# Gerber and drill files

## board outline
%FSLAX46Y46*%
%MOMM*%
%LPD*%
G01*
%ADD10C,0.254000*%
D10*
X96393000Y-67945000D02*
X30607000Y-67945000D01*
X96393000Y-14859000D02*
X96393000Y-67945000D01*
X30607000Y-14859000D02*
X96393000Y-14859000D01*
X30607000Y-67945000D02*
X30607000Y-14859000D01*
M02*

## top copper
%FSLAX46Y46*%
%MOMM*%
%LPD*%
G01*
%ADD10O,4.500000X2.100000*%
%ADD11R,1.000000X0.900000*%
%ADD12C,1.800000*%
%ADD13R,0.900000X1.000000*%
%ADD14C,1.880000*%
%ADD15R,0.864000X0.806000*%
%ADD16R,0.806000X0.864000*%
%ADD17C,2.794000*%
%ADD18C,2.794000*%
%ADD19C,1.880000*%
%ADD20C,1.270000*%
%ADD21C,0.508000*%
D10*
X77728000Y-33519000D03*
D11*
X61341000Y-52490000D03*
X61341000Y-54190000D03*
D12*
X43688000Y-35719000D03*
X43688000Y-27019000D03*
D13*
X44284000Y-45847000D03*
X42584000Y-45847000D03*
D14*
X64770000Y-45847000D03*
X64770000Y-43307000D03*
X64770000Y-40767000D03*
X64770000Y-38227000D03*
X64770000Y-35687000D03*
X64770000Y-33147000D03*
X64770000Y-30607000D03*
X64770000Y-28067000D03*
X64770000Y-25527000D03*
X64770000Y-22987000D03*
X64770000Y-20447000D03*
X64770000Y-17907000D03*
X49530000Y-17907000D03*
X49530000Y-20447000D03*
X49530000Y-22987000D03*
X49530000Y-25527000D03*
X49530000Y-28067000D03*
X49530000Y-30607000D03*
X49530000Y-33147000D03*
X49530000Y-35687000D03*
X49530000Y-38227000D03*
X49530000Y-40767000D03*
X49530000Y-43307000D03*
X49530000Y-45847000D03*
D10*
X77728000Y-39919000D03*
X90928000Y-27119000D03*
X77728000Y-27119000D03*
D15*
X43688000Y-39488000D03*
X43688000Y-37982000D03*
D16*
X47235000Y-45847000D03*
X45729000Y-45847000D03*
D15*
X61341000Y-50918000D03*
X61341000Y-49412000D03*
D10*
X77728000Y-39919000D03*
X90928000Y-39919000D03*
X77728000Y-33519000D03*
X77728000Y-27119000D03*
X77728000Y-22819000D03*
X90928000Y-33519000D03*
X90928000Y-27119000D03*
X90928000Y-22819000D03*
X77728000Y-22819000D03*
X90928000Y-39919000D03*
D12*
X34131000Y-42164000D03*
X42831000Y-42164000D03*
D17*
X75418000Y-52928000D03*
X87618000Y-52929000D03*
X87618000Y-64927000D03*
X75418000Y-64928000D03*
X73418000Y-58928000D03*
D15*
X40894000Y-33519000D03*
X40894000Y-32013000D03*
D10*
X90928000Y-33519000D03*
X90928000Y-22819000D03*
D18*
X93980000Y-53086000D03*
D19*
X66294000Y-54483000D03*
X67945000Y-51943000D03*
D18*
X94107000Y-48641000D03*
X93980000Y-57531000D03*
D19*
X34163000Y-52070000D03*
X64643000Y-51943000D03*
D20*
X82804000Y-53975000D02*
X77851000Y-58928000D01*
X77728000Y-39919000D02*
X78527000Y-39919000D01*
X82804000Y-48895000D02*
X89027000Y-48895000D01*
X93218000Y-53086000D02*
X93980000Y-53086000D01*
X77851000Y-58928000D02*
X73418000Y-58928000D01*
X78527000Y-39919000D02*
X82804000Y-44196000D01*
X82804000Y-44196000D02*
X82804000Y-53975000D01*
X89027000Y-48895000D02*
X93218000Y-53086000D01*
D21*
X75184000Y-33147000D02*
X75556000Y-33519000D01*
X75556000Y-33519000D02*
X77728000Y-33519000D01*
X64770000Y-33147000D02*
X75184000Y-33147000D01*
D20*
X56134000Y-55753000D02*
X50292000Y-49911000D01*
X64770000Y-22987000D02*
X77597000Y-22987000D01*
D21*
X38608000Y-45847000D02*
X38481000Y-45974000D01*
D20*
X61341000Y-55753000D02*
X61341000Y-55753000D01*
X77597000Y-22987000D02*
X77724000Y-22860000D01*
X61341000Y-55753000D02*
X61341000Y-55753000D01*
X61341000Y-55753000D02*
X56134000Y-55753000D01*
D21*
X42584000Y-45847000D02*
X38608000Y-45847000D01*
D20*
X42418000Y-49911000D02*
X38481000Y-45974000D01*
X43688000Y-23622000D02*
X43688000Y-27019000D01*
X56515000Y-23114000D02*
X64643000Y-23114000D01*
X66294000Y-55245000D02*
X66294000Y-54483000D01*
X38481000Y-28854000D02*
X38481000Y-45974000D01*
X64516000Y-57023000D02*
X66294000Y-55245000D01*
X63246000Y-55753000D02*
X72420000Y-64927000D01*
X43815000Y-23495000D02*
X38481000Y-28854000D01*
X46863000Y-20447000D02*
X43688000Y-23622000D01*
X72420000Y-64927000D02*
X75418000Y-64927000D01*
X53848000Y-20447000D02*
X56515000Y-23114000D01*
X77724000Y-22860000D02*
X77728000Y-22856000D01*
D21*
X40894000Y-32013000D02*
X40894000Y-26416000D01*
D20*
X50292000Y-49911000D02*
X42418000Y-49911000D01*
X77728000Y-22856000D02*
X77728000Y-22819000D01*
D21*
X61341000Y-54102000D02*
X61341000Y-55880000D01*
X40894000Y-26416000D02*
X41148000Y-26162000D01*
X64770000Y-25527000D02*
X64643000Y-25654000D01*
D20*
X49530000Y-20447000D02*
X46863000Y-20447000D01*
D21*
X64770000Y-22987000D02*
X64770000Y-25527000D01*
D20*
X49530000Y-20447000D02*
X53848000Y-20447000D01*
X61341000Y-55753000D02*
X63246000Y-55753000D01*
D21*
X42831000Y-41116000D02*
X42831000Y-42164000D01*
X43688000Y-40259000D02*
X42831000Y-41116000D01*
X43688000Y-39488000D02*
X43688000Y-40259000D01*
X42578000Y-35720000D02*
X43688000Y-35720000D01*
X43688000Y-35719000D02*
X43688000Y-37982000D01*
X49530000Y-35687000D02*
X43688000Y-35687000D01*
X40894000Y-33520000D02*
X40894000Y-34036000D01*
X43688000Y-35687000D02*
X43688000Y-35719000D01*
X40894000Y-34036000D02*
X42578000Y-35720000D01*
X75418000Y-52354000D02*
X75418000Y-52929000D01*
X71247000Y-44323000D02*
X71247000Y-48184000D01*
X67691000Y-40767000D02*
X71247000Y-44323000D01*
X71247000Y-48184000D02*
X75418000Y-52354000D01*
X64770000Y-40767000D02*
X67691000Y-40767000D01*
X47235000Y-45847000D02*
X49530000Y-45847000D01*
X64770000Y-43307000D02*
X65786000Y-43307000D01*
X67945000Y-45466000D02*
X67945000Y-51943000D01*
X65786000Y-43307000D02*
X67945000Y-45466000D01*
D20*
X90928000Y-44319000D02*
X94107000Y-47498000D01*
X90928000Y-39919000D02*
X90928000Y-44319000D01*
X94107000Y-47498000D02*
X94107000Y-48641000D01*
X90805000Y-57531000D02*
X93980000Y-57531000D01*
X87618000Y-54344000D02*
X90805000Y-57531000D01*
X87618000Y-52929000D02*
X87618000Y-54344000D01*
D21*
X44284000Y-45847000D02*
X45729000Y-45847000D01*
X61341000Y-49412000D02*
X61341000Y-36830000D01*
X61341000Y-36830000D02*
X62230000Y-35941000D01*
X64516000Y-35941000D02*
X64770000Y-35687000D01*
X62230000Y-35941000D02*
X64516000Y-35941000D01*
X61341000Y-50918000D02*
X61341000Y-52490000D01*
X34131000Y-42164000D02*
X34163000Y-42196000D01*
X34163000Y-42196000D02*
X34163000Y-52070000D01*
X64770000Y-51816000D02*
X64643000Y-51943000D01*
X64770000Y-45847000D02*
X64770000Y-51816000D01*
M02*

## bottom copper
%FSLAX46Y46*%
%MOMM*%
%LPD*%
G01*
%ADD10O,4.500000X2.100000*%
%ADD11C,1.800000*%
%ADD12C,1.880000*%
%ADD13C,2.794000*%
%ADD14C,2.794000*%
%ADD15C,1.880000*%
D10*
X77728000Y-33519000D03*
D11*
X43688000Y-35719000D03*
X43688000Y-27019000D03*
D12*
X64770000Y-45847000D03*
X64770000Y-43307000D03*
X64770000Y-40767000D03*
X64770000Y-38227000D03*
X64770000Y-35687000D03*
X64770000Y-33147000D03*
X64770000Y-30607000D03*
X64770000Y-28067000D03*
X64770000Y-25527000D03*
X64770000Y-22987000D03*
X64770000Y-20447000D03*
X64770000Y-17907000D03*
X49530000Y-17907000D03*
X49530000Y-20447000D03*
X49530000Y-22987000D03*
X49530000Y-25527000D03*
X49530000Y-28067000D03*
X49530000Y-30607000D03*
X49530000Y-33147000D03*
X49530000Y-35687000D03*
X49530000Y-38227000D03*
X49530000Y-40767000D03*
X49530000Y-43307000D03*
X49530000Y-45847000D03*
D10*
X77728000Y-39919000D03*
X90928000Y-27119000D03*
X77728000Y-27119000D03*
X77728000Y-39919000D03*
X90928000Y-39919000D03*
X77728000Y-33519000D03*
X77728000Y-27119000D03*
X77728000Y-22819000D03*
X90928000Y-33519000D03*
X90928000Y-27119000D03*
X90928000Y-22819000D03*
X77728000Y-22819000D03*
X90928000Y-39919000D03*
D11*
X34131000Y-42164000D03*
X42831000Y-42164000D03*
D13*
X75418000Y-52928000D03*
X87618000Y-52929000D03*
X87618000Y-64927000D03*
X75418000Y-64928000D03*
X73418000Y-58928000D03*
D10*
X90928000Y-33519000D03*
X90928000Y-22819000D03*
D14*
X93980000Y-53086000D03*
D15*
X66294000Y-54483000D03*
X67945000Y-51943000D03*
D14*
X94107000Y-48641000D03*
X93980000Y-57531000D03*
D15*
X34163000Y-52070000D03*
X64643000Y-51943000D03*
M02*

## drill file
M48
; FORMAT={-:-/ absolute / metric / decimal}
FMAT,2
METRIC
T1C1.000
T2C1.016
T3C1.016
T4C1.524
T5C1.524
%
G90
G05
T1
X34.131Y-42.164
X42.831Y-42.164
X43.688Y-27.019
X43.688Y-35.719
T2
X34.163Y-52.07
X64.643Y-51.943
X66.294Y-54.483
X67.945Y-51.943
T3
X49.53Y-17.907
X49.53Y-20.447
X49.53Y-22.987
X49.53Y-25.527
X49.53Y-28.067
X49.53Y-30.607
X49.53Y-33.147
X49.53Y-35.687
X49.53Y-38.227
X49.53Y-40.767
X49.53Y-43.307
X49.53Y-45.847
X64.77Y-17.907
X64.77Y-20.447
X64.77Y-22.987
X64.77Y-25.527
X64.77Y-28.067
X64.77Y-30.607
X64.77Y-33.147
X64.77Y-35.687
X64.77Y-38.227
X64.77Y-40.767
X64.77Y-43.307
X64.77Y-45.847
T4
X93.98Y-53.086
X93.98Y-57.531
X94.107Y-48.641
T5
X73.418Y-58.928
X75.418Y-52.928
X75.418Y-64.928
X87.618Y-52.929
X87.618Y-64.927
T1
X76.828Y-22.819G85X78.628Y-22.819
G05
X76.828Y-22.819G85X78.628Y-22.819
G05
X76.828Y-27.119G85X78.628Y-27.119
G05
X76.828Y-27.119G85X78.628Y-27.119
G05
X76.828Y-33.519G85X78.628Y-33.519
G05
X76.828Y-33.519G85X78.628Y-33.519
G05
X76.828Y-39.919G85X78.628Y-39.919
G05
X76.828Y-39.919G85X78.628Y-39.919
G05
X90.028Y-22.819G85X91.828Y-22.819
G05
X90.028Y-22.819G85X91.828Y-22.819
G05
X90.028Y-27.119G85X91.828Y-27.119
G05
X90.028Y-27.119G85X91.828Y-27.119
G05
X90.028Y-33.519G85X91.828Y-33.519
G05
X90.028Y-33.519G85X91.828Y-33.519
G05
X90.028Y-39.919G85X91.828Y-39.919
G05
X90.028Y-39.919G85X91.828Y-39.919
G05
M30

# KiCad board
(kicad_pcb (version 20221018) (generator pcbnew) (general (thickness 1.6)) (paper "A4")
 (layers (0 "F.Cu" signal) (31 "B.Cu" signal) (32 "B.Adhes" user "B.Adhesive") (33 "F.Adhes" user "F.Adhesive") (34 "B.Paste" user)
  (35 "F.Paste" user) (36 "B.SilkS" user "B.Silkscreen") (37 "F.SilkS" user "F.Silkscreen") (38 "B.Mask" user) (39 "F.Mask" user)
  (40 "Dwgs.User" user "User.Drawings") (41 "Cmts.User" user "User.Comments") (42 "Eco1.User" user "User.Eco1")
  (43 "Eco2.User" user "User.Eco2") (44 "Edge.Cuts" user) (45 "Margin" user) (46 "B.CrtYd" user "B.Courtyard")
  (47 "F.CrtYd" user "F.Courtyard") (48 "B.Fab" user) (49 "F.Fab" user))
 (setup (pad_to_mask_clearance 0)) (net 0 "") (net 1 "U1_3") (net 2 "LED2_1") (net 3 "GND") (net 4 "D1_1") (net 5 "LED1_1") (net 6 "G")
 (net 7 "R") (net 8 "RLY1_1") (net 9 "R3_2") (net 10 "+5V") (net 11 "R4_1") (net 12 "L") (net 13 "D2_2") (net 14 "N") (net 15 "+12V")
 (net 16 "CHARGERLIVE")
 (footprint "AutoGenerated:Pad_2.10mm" (layer "F.Cu") (at 77.728 33.519)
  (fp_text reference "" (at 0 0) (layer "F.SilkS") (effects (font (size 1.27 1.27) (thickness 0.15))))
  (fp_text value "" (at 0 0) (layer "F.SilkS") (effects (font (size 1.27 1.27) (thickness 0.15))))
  (pad "5" thru_hole oval (at 0 0 90) (size 2.1 4.5) (drill oval 1 2.8) (layers "*.Cu" "*.Paste" "*.Mask") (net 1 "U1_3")))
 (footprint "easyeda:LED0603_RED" (layer "F.Cu") (at 61.341 53.34 -90)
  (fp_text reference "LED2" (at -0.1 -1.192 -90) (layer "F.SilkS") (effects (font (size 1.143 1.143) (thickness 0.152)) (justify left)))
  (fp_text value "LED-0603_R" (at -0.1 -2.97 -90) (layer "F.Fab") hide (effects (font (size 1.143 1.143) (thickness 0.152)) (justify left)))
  (pad "1" smd rect (at -0.85 0 180) (size 1 0.9) (layers "F.Cu" "F.Paste" "F.Mask") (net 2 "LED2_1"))
  (pad "2" smd rect (at 0.85 0 180) (size 1 0.9) (layers "F.Cu" "F.Paste" "F.Mask") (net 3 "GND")))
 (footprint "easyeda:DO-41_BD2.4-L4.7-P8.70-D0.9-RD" (layer "F.Cu") (at 43.688 31.369 -90)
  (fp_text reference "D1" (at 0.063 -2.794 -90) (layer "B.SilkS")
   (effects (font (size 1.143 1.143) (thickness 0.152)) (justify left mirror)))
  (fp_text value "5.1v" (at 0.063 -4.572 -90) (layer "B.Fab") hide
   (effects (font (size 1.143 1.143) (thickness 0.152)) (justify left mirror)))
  (pad "1" thru_hole circle (at 4.35 0 270) (size 1.8 1.8) (drill 1) (layers "*.Cu" "*.Paste" "*.Mask") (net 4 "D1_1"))
  (pad "2" thru_hole circle (at -4.35 0 270) (size 1.8 1.8) (drill 1) (layers "*.Cu" "*.Paste" "*.Mask") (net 3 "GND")))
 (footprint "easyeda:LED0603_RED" (layer "F.Cu") (at 43.434 45.847 180)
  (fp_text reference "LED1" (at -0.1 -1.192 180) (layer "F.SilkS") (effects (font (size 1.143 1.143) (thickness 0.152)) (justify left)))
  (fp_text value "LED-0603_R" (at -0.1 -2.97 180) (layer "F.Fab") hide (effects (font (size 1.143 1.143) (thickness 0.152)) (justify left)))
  (pad "1" smd rect (at -0.85 0 90) (size 1 0.9) (layers "F.Cu" "F.Paste" "F.Mask") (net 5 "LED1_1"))
  (pad "2" smd rect (at 0.85 0 90) (size 1 0.9) (layers "F.Cu" "F.Paste" "F.Mask") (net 3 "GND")))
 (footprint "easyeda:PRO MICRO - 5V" (layer "F.Cu") (at 57.15 31.877)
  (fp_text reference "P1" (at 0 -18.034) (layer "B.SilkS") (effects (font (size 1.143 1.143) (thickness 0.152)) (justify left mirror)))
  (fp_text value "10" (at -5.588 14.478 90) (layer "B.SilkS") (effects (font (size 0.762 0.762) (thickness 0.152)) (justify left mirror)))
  (pad "1" thru_hole circle (at 7.62 13.97) (size 1.88 1.88) (drill 1.016) (layers "*.Cu" "*.Paste" "*.Mask") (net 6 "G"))
  (pad "2" thru_hole circle (at 7.62 11.43) (size 1.88 1.88) (drill 1.016) (layers "*.Cu" "*.Paste" "*.Mask") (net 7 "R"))
  (pad "3" thru_hole circle (at 7.62 8.89) (size 1.88 1.88) (drill 1.016) (layers "*.Cu" "*.Paste" "*.Mask") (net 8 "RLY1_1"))
  (pad "4" thru_hole circle (at 7.62 6.35) (size 1.88 1.88) (drill 1.016) (layers "*.Cu" "*.Paste" "*.Mask"))
  (pad "5" thru_hole circle (at 7.62 3.81) (size 1.88 1.88) (drill 1.016) (layers "*.Cu" "*.Paste" "*.Mask") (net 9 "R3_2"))
  (pad "6" thru_hole circle (at 7.62 1.27) (size 1.88 1.88) (drill 1.016) (layers "*.Cu" "*.Paste" "*.Mask") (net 1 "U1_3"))
  (pad "7" thru_hole circle (at 7.62 -1.27) (size 1.88 1.88) (drill 1.016) (layers "*.Cu" "*.Paste" "*.Mask"))
  (pad "8" thru_hole circle (at 7.62 -3.81) (size 1.88 1.88) (drill 1.016) (layers "*.Cu" "*.Paste" "*.Mask"))
  (pad "9" thru_hole circle (at 7.62 -6.35) (size 1.88 1.88) (drill 1.016) (layers "*.Cu" "*.Paste" "*.Mask") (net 3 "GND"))
  (pad "10" thru_hole circle (at 7.62 -8.89) (size 1.88 1.88) (drill 1.016) (layers "*.Cu" "*.Paste" "*.Mask") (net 3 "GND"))
  (pad "11" thru_hole circle (at 7.62 -11.43) (size 1.88 1.88) (drill 1.016) (layers "*.Cu" "*.Paste" "*.Mask"))
  (pad "12" thru_hole circle (at 7.62 -13.97) (size 1.88 1.88) (drill 1.016) (layers "*.Cu" "*.Paste" "*.Mask"))
  (pad "13" thru_hole circle (at -7.62 -13.97 180) (size 1.88 1.88) (drill 1.016) (layers "*.Cu" "*.Paste" "*.Mask"))
  (pad "14" thru_hole circle (at -7.62 -11.43 180) (size 1.88 1.88) (drill 1.016) (layers "*.Cu" "*.Paste" "*.Mask") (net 3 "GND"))
  (pad "15" thru_hole circle (at -7.62 -8.89 180) (size 1.88 1.88) (drill 1.016) (layers "*.Cu" "*.Paste" "*.Mask"))
  (pad "16" thru_hole circle (at -7.62 -6.35 180) (size 1.88 1.88) (drill 1.016) (layers "*.Cu" "*.Paste" "*.Mask") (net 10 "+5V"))
  (pad "17" thru_hole circle (at -7.62 -3.81 180) (size 1.88 1.88) (drill 1.016) (layers "*.Cu" "*.Paste" "*.Mask"))
  (pad "18" thru_hole circle (at -7.62 -1.27 180) (size 1.88 1.88) (drill 1.016) (layers "*.Cu" "*.Paste" "*.Mask"))
  (pad "19" thru_hole circle (at -7.62 1.27 180) (size 1.88 1.88) (drill 1.016) (layers "*.Cu" "*.Paste" "*.Mask"))
  (pad "20" thru_hole circle (at -7.62 3.81 180) (size 1.88 1.88) (drill 1.016) (layers "*.Cu" "*.Paste" "*.Mask") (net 4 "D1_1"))
  (pad "21" thru_hole circle (at -7.62 6.35 180) (size 1.88 1.88) (drill 1.016) (layers "*.Cu" "*.Paste" "*.Mask"))
  (pad "22" thru_hole circle (at -7.62 8.89 180) (size 1.88 1.88) (drill 1.016) (layers "*.Cu" "*.Paste" "*.Mask"))
  (pad "23" thru_hole circle (at -7.62 11.43 180) (size 1.88 1.88) (drill 1.016) (layers "*.Cu" "*.Paste" "*.Mask"))
  (pad "24" thru_hole circle (at -7.62 13.97 180) (size 1.88 1.88) (drill 1.016) (layers "*.Cu" "*.Paste" "*.Mask") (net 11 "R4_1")))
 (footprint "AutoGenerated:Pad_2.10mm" (layer "F.Cu") (at 77.728 39.919)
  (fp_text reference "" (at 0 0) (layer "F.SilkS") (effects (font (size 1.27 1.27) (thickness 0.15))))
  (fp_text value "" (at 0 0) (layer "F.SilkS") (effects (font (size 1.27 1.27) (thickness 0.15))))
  (pad "5" thru_hole oval (at 0 0 90) (size 2.1 4.5) (drill oval 1 2.8) (layers "*.Cu" "*.Paste" "*.Mask") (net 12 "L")))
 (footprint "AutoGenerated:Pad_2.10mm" (layer "F.Cu") (at 90.928 27.119)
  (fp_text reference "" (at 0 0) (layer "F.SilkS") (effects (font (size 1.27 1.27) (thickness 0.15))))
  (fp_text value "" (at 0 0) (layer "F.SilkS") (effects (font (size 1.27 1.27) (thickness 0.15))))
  (pad "5" thru_hole oval (at 0 0 90) (size 2.1 4.5) (drill oval 1 2.8) (layers "*.Cu" "*.Paste" "*.Mask")))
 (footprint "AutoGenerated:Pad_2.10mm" (layer "F.Cu") (at 77.728 27.119)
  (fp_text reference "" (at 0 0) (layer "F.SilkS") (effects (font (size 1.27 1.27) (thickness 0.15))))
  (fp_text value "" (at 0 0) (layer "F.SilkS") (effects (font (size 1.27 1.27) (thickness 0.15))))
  (pad "5" thru_hole oval (at 0 0 90) (size 2.1 4.5) (drill oval 1 2.8) (layers "*.Cu" "*.Paste" "*.Mask")))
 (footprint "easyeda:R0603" (layer "F.Cu") (at 43.688 38.735 90)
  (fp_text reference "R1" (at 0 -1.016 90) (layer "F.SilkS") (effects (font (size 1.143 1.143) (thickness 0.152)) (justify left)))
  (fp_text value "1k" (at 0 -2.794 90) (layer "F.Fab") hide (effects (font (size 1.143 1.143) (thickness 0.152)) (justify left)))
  (pad "1" smd rect (at -0.753 0 90) (size 0.806 0.864) (layers "F.Cu" "F.Paste" "F.Mask") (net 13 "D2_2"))
  (pad "2" smd rect (at 0.753 0 90) (size 0.806 0.864) (layers "F.Cu" "F.Paste" "F.Mask") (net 4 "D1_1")))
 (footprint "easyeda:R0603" (layer "F.Cu") (at 46.482 45.847 180)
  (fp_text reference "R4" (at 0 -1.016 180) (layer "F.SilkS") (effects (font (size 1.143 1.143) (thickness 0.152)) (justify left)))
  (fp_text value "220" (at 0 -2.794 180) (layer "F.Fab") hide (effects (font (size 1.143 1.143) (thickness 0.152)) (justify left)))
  (pad "1" smd rect (at -0.753 0 180) (size 0.806 0.864) (layers "F.Cu" "F.Paste" "F.Mask") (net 11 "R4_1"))
  (pad "2" smd rect (at 0.753 0 180) (size 0.806 0.864) (layers "F.Cu" "F.Paste" "F.Mask") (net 5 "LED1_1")))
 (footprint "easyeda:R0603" (layer "F.Cu") (at 61.341 50.165 90)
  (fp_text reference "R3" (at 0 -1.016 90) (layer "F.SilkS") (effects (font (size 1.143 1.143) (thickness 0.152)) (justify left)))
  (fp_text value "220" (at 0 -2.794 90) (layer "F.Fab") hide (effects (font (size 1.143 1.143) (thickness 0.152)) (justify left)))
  (pad "1" smd rect (at -0.753 0 90) (size 0.806 0.864) (layers "F.Cu" "F.Paste" "F.Mask") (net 2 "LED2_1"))
  (pad "2" smd rect (at 0.753 0 90) (size 0.806 0.864) (layers "F.Cu" "F.Paste" "F.Mask") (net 9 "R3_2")))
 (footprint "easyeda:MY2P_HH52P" (layer "F.Cu") (at 84.328 31.369 90)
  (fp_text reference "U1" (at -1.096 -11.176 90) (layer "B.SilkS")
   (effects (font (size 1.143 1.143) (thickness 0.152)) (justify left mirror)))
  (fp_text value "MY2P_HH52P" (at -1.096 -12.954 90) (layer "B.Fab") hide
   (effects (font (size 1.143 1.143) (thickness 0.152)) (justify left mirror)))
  (pad "1" thru_hole oval (at -8.55 -6.6 90) (size 2.1 4.5) (drill oval 1 2.8) (layers "*.Cu" "*.Paste" "*.Mask") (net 12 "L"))
  (pad "2" thru_hole oval (at -8.55 6.6 90) (size 2.1 4.5) (drill oval 1 2.8) (layers "*.Cu" "*.Paste" "*.Mask") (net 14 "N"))
  (pad "3" thru_hole oval (at -2.15 -6.6 90) (size 2.1 4.5) (drill oval 1 2.8) (layers "*.Cu" "*.Paste" "*.Mask") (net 1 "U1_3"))
  (pad "4" thru_hole oval (at 4.25 -6.6 90) (size 2.1 4.5) (drill oval 1 2.8) (layers "*.Cu" "*.Paste" "*.Mask"))
  (pad "5" thru_hole oval (at 8.55 -6.6 90) (size 2.1 4.5) (drill oval 1 2.8) (layers "*.Cu" "*.Paste" "*.Mask") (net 3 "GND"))
  (pad "6" thru_hole oval (at -2.15 6.6 90) (size 2.1 4.5) (drill oval 1 2.8) (layers "*.Cu" "*.Paste" "*.Mask"))
  (pad "7" thru_hole oval (at 4.25 6.6 90) (size 2.1 4.5) (drill oval 1 2.8) (layers "*.Cu" "*.Paste" "*.Mask"))
  (pad "8" thru_hole oval (at 8.55 6.6 90) (size 2.1 4.5) (drill oval 1 2.8) (layers "*.Cu" "*.Paste" "*.Mask")))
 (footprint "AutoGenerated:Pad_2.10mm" (layer "F.Cu") (at 77.728 22.819)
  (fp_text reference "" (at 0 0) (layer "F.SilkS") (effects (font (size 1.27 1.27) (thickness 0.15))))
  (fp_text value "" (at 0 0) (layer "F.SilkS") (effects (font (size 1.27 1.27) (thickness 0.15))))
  (pad "5" thru_hole oval (at 0 0 90) (size 2.1 4.5) (drill oval 1 2.8) (layers "*.Cu" "*.Paste" "*.Mask") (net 3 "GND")))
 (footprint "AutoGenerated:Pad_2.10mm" (layer "F.Cu") (at 90.928 39.919)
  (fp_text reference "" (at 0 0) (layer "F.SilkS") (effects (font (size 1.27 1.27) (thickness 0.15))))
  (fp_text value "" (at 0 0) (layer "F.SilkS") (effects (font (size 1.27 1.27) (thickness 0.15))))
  (pad "5" thru_hole oval (at 0 0 90) (size 2.1 4.5) (drill oval 1 2.8) (layers "*.Cu" "*.Paste" "*.Mask") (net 14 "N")))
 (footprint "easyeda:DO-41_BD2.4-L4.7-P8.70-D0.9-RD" (layer "F.Cu") (at 38.481 42.164 180)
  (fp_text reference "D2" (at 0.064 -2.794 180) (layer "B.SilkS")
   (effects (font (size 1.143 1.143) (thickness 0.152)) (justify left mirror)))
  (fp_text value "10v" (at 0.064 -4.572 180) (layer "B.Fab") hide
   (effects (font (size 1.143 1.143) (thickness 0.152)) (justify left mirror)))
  (pad "1" thru_hole circle (at 4.35 0 180) (size 1.8 1.8) (drill 1) (layers "*.Cu" "*.Paste" "*.Mask") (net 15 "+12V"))
  (pad "2" thru_hole circle (at -4.35 0 180) (size 1.8 1.8) (drill 1) (layers "*.Cu" "*.Paste" "*.Mask") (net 13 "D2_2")))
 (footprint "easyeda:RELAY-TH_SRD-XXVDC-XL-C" (layer "F.Cu") (at 80.518 58.928 180)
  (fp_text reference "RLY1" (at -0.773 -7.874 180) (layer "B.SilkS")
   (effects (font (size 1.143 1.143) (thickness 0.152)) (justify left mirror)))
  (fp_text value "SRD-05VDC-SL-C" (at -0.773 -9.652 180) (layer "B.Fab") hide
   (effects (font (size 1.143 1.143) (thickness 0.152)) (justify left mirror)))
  (pad "1" thru_hole circle (at 5.1 6) (size 2.794 2.794) (drill 1.524) (layers "*.Cu" "*.Paste" "*.Mask") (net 8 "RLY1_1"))
  (pad "2" thru_hole circle (at -7.1 5.999) (size 2.794 2.794) (drill 1.524) (layers "*.Cu" "*.Paste" "*.Mask") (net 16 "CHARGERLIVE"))
  (pad "3" thru_hole circle (at -7.1 -5.999) (size 2.794 2.794) (drill 1.524) (layers "*.Cu" "*.Paste" "*.Mask"))
  (pad "4" thru_hole circle (at 5.1 -6) (size 2.794 2.794) (drill 1.524) (layers "*.Cu" "*.Paste" "*.Mask") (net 3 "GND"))
  (pad "5" thru_hole circle (at 7.1 0) (size 2.794 2.794) (drill 1.524) (layers "*.Cu" "*.Paste" "*.Mask") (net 12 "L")))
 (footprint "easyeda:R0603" (layer "F.Cu") (at 40.894 32.766 90)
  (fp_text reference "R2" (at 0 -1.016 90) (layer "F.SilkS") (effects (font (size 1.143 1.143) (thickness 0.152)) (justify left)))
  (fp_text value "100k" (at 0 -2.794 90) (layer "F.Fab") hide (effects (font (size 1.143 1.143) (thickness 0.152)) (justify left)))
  (pad "1" smd rect (at -0.753 0 90) (size 0.806 0.864) (layers "F.Cu" "F.Paste" "F.Mask") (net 4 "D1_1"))
  (pad "2" smd rect (at 0.753 0 90) (size 0.806 0.864) (layers "F.Cu" "F.Paste" "F.Mask") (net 3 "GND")))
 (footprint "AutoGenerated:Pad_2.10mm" (layer "F.Cu") (at 90.928 33.519)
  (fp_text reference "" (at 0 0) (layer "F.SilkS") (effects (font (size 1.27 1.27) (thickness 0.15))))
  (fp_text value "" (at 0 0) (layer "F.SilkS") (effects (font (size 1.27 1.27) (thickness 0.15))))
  (pad "5" thru_hole oval (at 0 0 90) (size 2.1 4.5) (drill oval 1 2.8) (layers "*.Cu" "*.Paste" "*.Mask")))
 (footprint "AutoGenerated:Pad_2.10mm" (layer "F.Cu") (at 90.928 22.819)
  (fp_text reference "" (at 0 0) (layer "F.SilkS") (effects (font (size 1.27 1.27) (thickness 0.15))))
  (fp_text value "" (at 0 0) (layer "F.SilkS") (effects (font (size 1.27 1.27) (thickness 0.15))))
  (pad "5" thru_hole oval (at 0 0 90) (size 2.1 4.5) (drill oval 1 2.8) (layers "*.Cu" "*.Paste" "*.Mask")))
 (gr_line (start 96.393 67.945) (end 30.607 67.945) (stroke (width 0.254) (type solid)) (layer "Edge.Cuts"))
 (gr_line (start 96.393 14.859) (end 96.393 67.945) (stroke (width 0.254) (type solid)) (layer "Edge.Cuts"))
 (gr_line (start 30.607 14.859) (end 96.393 14.859) (stroke (width 0.254) (type solid)) (layer "Edge.Cuts"))
 (gr_line (start 30.607 67.945) (end 30.607 14.859) (stroke (width 0.254) (type solid)) (layer "Edge.Cuts"))
 (segment (start 82.804 53.975) (end 77.851 58.928) (width 1.27) (layer "F.Cu") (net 12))
 (segment (start 77.728 39.919) (end 78.527 39.919) (width 1.27) (layer "F.Cu") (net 12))
 (segment (start 82.804 48.895) (end 89.027 48.895) (width 1.27) (layer "F.Cu") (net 12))
 (segment (start 93.218 53.086) (end 93.98 53.086) (width 1.27) (layer "F.Cu") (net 12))
 (segment (start 77.851 58.928) (end 73.418 58.928) (width 1.27) (layer "F.Cu") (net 12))
 (segment (start 78.527 39.919) (end 82.804 44.196) (width 1.27) (layer "F.Cu") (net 12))
 (segment (start 82.804 44.196) (end 82.804 53.975) (width 1.27) (layer "F.Cu") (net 12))
 (segment (start 89.027 48.895) (end 93.218 53.086) (width 1.27) (layer "F.Cu") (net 12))
 (via (at 93.98 53.086) (size 2.794) (drill 1.524) (layers "F.Cu" "B.Cu") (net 12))
 (segment (start 75.184 33.147) (end 75.556 33.519) (width 0.508) (layer "F.Cu") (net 1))
 (segment (start 75.556 33.519) (end 77.728 33.519) (width 0.508) (layer "F.Cu") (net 1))
 (segment (start 64.77 33.147) (end 75.184 33.147) (width 0.508) (layer "F.Cu") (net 1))
 (segment (start 56.134 55.753) (end 50.292 49.911) (width 1.27) (layer "F.Cu") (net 3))
 (segment (start 64.77 22.987) (end 77.597 22.987) (width 1.27) (layer "F.Cu") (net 3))
 (segment (start 38.608 45.847) (end 38.481 45.974) (width 0.508) (layer "F.Cu") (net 3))
 (segment (start 61.341 55.753) (end 61.341 55.753) (width 1.27) (layer "F.Cu") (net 3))
 (segment (start 77.597 22.987) (end 77.724 22.86) (width 1.27) (layer "F.Cu") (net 3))
 (segment (start 61.341 55.753) (end 61.341 55.753) (width 1.27) (layer "F.Cu") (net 3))
 (segment (start 61.341 55.753) (end 56.134 55.753) (width 1.27) (layer "F.Cu") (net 3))
 (segment (start 42.584 45.847) (end 38.608 45.847) (width 0.508) (layer "F.Cu") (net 3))
 (segment (start 42.418 49.911) (end 38.481 45.974) (width 1.27) (layer "F.Cu") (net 3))
 (segment (start 43.688 23.622) (end 43.688 27.019) (width 1.27) (layer "F.Cu") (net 3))
 (segment (start 56.515 23.114) (end 64.643 23.114) (width 1.27) (layer "F.Cu") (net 3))
 (segment (start 66.294 55.245) (end 66.294 54.483) (width 1.27) (layer "F.Cu") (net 3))
 (segment (start 38.481 28.854) (end 38.481 45.974) (width 1.27) (layer "F.Cu") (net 3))
 (segment (start 64.516 57.023) (end 66.294 55.245) (width 1.27) (layer "F.Cu") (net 3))
 (segment (start 63.246 55.753) (end 72.42 64.927) (width 1.27) (layer "F.Cu") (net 3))
 (segment (start 43.815 23.495) (end 38.481 28.854) (width 1.27) (layer "F.Cu") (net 3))
 (segment (start 46.863 20.447) (end 43.688 23.622) (width 1.27) (layer "F.Cu") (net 3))
 (segment (start 72.42 64.927) (end 75.418 64.927) (width 1.27) (layer "F.Cu") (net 3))
 (segment (start 53.848 20.447) (end 56.515 23.114) (width 1.27) (layer "F.Cu") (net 3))
 (segment (start 77.724 22.86) (end 77.728 22.856) (width 1.27) (layer "F.Cu") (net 3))
 (segment (start 40.894 32.013) (end 40.894 26.416) (width 0.508) (layer "F.Cu") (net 3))
 (segment (start 50.292 49.911) (end 42.418 49.911) (width 1.27) (layer "F.Cu") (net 3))
 (segment (start 77.728 22.856) (end 77.728 22.819) (width 1.27) (layer "F.Cu") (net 3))
 (segment (start 61.341 54.102) (end 61.341 55.88) (width 0.508) (layer "F.Cu") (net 3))
 (segment (start 40.894 26.416) (end 41.148 26.162) (width 0.508) (layer "F.Cu") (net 3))
 (segment (start 64.77 25.527) (end 64.643 25.654) (width 0.508) (layer "F.Cu") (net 3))
 (segment (start 49.53 20.447) (end 46.863 20.447) (width 1.27) (layer "F.Cu") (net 3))
 (segment (start 64.77 22.987) (end 64.77 25.527) (width 0.508) (layer "F.Cu") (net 3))
 (segment (start 49.53 20.447) (end 53.848 20.447) (width 1.27) (layer "F.Cu") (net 3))
 (segment (start 61.341 55.753) (end 63.246 55.753) (width 1.27) (layer "F.Cu") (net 3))
 (via (at 66.294 54.483) (size 1.88) (drill 1.016) (layers "F.Cu" "B.Cu") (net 3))
 (segment (start 42.831 41.116) (end 42.831 42.164) (width 0.508) (layer "F.Cu") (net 13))
 (segment (start 43.688 40.259) (end 42.831 41.116) (width 0.508) (layer "F.Cu") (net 13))
 (segment (start 43.688 39.488) (end 43.688 40.259) (width 0.508) (layer "F.Cu") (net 13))
 (segment (start 42.578 35.72) (end 43.688 35.72) (width 0.508) (layer "F.Cu") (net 4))
 (segment (start 43.688 35.719) (end 43.688 37.982) (width 0.508) (layer "F.Cu") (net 4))
 (segment (start 49.53 35.687) (end 43.688 35.687) (width 0.508) (layer "F.Cu") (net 4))
 (segment (start 40.894 33.52) (end 40.894 34.036) (width 0.508) (layer "F.Cu") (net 4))
 (segment (start 43.688 35.687) (end 43.688 35.719) (width 0.508) (layer "F.Cu") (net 4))
 (segment (start 40.894 34.036) (end 42.578 35.72) (width 0.508) (layer "F.Cu") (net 4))
 (segment (start 75.418 52.354) (end 75.418 52.929) (width 0.508) (layer "F.Cu") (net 8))
 (segment (start 71.247 44.323) (end 71.247 48.184) (width 0.508) (layer "F.Cu") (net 8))
 (segment (start 67.691 40.767) (end 71.247 44.323) (width 0.508) (layer "F.Cu") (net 8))
 (segment (start 71.247 48.184) (end 75.418 52.354) (width 0.508) (layer "F.Cu") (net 8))
 (segment (start 64.77 40.767) (end 67.691 40.767) (width 0.508) (layer "F.Cu") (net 8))
 (segment (start 47.235 45.847) (end 49.53 45.847) (width 0.508) (layer "F.Cu") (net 11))
 (segment (start 64.77 43.307) (end 65.786 43.307) (width 0.508) (layer "F.Cu") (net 7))
 (segment (start 67.945 45.466) (end 67.945 51.943) (width 0.508) (layer "F.Cu") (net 7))
 (segment (start 65.786 43.307) (end 67.945 45.466) (width 0.508) (layer "F.Cu") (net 7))
 (via (at 67.945 51.943) (size 1.88) (drill 1.016) (layers "F.Cu" "B.Cu") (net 7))
 (segment (start 90.928 44.319) (end 94.107 47.498) (width 1.27) (layer "F.Cu") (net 14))
 (segment (start 90.928 39.919) (end 90.928 44.319) (width 1.27) (layer "F.Cu") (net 14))
 (segment (start 94.107 47.498) (end 94.107 48.641) (width 1.27) (layer "F.Cu") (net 14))
 (via (at 94.107 48.641) (size 2.794) (drill 1.524) (layers "F.Cu" "B.Cu") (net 14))
 (segment (start 90.805 57.531) (end 93.98 57.531) (width 1.27) (layer "F.Cu") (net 16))
 (segment (start 87.618 54.344) (end 90.805 57.531) (width 1.27) (layer "F.Cu") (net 16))
 (segment (start 87.618 52.929) (end 87.618 54.344) (width 1.27) (layer "F.Cu") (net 16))
 (via (at 93.98 57.531) (size 2.794) (drill 1.524) (layers "F.Cu" "B.Cu") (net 16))
 (segment (start 44.284 45.847) (end 45.729 45.847) (width 0.508) (layer "F.Cu") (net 5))
 (segment (start 61.341 49.412) (end 61.341 36.83) (width 0.508) (layer "F.Cu") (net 9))
 (segment (start 61.341 36.83) (end 62.23 35.941) (width 0.508) (layer "F.Cu") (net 9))
 (segment (start 64.516 35.941) (end 64.77 35.687) (width 0.508) (layer "F.Cu") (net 9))
 (segment (start 62.23 35.941) (end 64.516 35.941) (width 0.508) (layer "F.Cu") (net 9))
 (segment (start 61.341 50.918) (end 61.341 52.49) (width 0.508) (layer "F.Cu") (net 2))
 (segment (start 34.131 42.164) (end 34.163 42.196) (width 0.508) (layer "F.Cu") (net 15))
 (segment (start 34.163 42.196) (end 34.163 52.07) (width 0.508) (layer "F.Cu") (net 15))
 (via (at 34.163 52.07) (size 1.88) (drill 1.016) (layers "F.Cu" "B.Cu") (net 15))
 (segment (start 64.77 51.816) (end 64.643 51.943) (width 0.508) (layer "F.Cu") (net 6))
 (segment (start 64.77 45.847) (end 64.77 51.816) (width 0.508) (layer "F.Cu") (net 6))
 (via (at 64.643 51.943) (size 1.88) (drill 1.016) (layers "F.Cu" "B.Cu") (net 6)))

